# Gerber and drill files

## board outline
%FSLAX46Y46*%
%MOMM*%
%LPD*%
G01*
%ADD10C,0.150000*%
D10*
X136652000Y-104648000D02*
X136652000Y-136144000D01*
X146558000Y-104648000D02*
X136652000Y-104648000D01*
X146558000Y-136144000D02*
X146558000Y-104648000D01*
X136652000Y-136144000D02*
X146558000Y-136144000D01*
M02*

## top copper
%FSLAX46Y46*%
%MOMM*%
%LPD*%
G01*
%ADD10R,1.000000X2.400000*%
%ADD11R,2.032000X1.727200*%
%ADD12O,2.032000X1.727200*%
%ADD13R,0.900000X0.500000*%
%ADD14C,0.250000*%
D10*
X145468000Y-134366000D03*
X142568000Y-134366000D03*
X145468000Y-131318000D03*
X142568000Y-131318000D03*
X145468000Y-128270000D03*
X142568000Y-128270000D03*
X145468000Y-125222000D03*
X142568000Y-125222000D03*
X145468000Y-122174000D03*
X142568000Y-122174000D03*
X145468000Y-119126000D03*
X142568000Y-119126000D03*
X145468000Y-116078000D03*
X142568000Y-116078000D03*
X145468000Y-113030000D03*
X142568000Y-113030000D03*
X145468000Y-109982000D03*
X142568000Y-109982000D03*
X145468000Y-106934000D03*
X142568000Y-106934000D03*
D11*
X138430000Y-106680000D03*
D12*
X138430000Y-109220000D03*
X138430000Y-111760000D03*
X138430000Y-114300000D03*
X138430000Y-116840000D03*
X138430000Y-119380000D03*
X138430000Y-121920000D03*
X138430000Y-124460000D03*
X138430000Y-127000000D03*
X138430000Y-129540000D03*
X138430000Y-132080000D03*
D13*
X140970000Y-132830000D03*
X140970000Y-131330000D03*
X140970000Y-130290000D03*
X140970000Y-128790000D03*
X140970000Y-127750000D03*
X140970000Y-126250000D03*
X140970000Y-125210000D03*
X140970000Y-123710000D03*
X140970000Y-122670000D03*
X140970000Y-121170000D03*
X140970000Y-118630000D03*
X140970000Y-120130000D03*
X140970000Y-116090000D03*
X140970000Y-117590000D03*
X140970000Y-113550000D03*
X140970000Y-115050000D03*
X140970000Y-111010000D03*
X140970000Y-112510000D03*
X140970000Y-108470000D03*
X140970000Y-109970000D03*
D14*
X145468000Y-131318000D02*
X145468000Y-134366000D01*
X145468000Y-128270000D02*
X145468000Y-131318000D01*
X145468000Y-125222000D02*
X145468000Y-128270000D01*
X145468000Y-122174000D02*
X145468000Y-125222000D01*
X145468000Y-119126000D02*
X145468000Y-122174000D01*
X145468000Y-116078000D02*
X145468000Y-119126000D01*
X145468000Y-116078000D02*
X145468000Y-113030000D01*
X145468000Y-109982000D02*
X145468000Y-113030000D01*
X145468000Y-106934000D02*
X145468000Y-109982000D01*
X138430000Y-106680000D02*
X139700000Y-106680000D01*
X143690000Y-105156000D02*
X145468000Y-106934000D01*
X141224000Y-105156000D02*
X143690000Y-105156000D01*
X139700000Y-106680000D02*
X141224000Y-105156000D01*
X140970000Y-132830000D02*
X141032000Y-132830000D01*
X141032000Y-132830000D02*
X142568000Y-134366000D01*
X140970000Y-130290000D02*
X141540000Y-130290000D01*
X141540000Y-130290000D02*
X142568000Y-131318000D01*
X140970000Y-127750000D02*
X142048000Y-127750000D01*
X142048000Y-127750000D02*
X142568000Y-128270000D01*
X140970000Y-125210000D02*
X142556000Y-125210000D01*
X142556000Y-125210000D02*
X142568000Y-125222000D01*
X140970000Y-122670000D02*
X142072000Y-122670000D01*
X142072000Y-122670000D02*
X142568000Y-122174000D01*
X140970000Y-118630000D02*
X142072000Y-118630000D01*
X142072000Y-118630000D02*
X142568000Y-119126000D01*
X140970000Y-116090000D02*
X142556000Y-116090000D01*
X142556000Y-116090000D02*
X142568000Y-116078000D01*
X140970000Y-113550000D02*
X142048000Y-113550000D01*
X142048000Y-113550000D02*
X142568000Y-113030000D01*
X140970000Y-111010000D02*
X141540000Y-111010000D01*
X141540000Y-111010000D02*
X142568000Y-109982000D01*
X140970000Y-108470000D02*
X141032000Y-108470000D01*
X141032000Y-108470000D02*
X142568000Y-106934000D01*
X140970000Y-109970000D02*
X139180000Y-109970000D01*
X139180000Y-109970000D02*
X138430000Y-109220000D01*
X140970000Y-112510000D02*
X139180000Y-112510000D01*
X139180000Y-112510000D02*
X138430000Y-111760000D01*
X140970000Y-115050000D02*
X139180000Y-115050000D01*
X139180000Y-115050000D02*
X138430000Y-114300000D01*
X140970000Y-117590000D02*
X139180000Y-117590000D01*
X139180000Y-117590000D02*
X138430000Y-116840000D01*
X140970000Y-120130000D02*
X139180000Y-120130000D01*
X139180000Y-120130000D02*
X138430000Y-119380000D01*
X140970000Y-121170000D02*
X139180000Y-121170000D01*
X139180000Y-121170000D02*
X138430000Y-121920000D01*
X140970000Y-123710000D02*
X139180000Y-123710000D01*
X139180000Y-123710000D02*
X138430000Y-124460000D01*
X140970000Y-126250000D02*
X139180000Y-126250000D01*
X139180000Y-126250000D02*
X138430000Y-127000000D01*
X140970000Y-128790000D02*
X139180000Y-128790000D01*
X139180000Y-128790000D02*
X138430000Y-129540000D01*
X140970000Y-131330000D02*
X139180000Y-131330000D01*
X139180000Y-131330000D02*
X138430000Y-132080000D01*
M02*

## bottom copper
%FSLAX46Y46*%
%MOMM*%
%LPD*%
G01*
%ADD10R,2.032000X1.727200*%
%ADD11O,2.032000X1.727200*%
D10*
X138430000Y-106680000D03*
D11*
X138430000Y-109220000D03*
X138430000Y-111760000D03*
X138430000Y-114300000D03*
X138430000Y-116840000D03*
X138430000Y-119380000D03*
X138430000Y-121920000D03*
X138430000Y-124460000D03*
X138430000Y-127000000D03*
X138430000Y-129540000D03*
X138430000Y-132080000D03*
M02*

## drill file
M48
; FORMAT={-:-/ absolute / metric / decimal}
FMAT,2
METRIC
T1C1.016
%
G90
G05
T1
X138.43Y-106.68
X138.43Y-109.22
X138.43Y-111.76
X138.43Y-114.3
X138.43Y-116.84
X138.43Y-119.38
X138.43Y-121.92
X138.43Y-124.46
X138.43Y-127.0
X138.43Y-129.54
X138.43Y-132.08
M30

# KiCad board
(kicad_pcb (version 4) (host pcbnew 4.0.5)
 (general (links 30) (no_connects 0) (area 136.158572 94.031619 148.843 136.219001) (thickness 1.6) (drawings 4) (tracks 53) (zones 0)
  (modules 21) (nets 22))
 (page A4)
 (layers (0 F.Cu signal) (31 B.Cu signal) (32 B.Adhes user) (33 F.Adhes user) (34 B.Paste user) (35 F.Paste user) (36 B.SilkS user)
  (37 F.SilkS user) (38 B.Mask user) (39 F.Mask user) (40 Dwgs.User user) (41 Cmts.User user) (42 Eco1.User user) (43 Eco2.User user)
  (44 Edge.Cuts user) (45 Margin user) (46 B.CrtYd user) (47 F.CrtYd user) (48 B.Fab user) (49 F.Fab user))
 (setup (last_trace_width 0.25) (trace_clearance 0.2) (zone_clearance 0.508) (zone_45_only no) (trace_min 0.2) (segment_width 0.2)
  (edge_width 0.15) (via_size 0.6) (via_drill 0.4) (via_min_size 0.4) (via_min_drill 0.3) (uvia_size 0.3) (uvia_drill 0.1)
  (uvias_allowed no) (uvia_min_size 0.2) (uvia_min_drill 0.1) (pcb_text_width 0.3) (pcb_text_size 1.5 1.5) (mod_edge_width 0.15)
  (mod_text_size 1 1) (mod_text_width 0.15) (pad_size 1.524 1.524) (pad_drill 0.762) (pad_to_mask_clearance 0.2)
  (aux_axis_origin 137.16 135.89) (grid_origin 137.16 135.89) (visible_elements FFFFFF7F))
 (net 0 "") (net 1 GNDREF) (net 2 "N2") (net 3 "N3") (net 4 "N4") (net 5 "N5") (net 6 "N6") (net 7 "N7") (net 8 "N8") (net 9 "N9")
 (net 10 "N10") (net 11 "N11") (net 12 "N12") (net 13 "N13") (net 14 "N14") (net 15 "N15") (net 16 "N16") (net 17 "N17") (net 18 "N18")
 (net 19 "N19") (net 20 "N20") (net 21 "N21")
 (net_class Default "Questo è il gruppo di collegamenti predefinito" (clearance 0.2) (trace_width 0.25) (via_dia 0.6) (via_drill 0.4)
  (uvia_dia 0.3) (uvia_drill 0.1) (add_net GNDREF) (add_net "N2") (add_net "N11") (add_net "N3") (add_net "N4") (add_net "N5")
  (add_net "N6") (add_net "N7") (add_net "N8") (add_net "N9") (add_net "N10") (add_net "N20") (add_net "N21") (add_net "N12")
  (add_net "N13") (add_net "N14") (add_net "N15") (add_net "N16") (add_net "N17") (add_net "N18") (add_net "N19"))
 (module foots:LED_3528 (layer F.Cu) (at 144.018 134.366 90)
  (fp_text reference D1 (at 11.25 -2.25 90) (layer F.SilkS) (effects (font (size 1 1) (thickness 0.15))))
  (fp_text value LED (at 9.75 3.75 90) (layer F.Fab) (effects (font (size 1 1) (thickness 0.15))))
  (pad 1 smd rect (at 0 1.45 90) (size 2.4 1) (layers F.Cu F.Paste F.Mask) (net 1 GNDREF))
  (pad 2 smd rect (at 0 -1.45 90) (size 2.4 1) (layers F.Cu F.Paste F.Mask) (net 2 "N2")))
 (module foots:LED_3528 (layer F.Cu) (at 144.018 131.318 90)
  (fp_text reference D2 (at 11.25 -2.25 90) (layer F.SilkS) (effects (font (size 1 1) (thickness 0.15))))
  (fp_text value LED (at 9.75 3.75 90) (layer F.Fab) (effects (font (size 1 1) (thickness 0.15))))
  (pad 1 smd rect (at 0 1.45 90) (size 2.4 1) (layers F.Cu F.Paste F.Mask) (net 1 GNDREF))
  (pad 2 smd rect (at 0 -1.45 90) (size 2.4 1) (layers F.Cu F.Paste F.Mask) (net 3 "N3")))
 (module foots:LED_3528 (layer F.Cu) (at 144.018 128.27 90)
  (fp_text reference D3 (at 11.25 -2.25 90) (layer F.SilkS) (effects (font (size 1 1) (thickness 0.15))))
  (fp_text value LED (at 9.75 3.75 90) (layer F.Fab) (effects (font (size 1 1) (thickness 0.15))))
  (pad 1 smd rect (at 0 1.45 90) (size 2.4 1) (layers F.Cu F.Paste F.Mask) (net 1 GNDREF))
  (pad 2 smd rect (at 0 -1.45 90) (size 2.4 1) (layers F.Cu F.Paste F.Mask) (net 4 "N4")))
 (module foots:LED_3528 (layer F.Cu) (at 144.018 125.222 90)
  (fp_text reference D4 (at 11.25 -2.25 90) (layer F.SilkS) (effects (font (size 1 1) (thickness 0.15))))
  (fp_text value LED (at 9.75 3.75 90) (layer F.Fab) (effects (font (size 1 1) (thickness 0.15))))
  (pad 1 smd rect (at 0 1.45 90) (size 2.4 1) (layers F.Cu F.Paste F.Mask) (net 1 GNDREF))
  (pad 2 smd rect (at 0 -1.45 90) (size 2.4 1) (layers F.Cu F.Paste F.Mask) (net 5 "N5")))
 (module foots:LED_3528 (layer F.Cu) (at 144.018 122.174 90)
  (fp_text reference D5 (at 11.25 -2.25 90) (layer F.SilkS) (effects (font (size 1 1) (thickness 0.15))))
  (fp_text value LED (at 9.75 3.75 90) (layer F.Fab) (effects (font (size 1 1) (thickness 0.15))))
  (pad 1 smd rect (at 0 1.45 90) (size 2.4 1) (layers F.Cu F.Paste F.Mask) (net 1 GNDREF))
  (pad 2 smd rect (at 0 -1.45 90) (size 2.4 1) (layers F.Cu F.Paste F.Mask) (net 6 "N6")))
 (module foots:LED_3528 (layer F.Cu) (at 144.018 119.126 90)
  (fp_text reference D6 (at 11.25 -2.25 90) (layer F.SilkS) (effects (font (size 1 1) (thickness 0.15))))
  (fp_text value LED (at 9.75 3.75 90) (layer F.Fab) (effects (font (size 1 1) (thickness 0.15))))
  (pad 1 smd rect (at 0 1.45 90) (size 2.4 1) (layers F.Cu F.Paste F.Mask) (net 1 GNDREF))
  (pad 2 smd rect (at 0 -1.45 90) (size 2.4 1) (layers F.Cu F.Paste F.Mask) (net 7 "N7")))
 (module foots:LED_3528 (layer F.Cu) (at 144.018 116.078 90)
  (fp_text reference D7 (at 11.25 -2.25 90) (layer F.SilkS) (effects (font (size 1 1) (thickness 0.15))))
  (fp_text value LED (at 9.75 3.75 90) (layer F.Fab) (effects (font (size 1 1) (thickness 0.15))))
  (pad 1 smd rect (at 0 1.45 90) (size 2.4 1) (layers F.Cu F.Paste F.Mask) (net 1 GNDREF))
  (pad 2 smd rect (at 0 -1.45 90) (size 2.4 1) (layers F.Cu F.Paste F.Mask) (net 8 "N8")))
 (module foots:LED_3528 (layer F.Cu) (at 144.018 113.03 90)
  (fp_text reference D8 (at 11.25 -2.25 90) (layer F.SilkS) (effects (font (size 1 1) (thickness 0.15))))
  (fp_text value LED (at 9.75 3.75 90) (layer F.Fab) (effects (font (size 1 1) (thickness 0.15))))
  (pad 1 smd rect (at 0 1.45 90) (size 2.4 1) (layers F.Cu F.Paste F.Mask) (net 1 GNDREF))
  (pad 2 smd rect (at 0 -1.45 90) (size 2.4 1) (layers F.Cu F.Paste F.Mask) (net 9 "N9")))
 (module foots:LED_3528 (layer F.Cu) (at 144.018 109.982 90)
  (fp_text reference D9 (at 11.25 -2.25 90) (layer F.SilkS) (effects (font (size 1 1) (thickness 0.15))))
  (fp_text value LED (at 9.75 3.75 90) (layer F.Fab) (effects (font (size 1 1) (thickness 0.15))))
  (pad 1 smd rect (at 0 1.45 90) (size 2.4 1) (layers F.Cu F.Paste F.Mask) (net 1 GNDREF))
  (pad 2 smd rect (at 0 -1.45 90) (size 2.4 1) (layers F.Cu F.Paste F.Mask) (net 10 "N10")))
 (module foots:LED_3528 (layer F.Cu) (at 144.018 106.934 90)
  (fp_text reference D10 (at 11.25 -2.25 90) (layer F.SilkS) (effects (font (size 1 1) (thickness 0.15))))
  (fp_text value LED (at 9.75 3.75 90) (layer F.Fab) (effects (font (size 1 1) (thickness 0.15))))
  (pad 1 smd rect (at 0 1.45 90) (size 2.4 1) (layers F.Cu F.Paste F.Mask) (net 1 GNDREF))
  (pad 2 smd rect (at 0 -1.45 90) (size 2.4 1) (layers F.Cu F.Paste F.Mask) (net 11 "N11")))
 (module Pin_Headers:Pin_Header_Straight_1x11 (layer F.Cu) (at 138.43 106.68)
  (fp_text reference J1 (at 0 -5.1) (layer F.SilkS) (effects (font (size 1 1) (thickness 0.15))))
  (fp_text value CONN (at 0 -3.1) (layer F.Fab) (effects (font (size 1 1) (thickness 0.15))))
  (pad 1 thru_hole rect (at 0 0) (size 2.032 1.7272) (drill 1.016) (layers *.Cu *.Mask) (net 1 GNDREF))
  (pad 2 thru_hole oval (at 0 2.54) (size 2.032 1.7272) (drill 1.016) (layers *.Cu *.Mask) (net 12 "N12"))
  (pad 3 thru_hole oval (at 0 5.08) (size 2.032 1.7272) (drill 1.016) (layers *.Cu *.Mask) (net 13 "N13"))
  (pad 4 thru_hole oval (at 0 7.62) (size 2.032 1.7272) (drill 1.016) (layers *.Cu *.Mask) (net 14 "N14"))
  (pad 5 thru_hole oval (at 0 10.16) (size 2.032 1.7272) (drill 1.016) (layers *.Cu *.Mask) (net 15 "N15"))
  (pad 6 thru_hole oval (at 0 12.7) (size 2.032 1.7272) (drill 1.016) (layers *.Cu *.Mask) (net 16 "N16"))
  (pad 7 thru_hole oval (at 0 15.24) (size 2.032 1.7272) (drill 1.016) (layers *.Cu *.Mask) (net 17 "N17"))
  (pad 8 thru_hole oval (at 0 17.78) (size 2.032 1.7272) (drill 1.016) (layers *.Cu *.Mask) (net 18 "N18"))
  (pad 9 thru_hole oval (at 0 20.32) (size 2.032 1.7272) (drill 1.016) (layers *.Cu *.Mask) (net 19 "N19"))
  (pad 10 thru_hole oval (at 0 22.86) (size 2.032 1.7272) (drill 1.016) (layers *.Cu *.Mask) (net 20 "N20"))
  (pad 11 thru_hole oval (at 0 25.4) (size 2.032 1.7272) (drill 1.016) (layers *.Cu *.Mask) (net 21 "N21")))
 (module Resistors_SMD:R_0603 (layer F.Cu) (at 140.97 132.08 90)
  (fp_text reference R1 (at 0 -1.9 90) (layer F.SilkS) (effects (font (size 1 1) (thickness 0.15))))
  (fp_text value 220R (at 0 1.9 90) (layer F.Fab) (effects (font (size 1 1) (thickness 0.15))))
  (pad 1 smd rect (at -0.75 0 90) (size 0.5 0.9) (layers F.Cu F.Paste F.Mask) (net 2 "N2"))
  (pad 2 smd rect (at 0.75 0 90) (size 0.5 0.9) (layers F.Cu F.Paste F.Mask) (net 21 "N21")))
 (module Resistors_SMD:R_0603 (layer F.Cu) (at 140.97 129.54 90)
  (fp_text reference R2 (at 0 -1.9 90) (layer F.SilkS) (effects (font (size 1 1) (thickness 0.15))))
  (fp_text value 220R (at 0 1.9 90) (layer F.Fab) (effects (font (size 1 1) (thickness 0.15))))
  (pad 1 smd rect (at -0.75 0 90) (size 0.5 0.9) (layers F.Cu F.Paste F.Mask) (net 3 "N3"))
  (pad 2 smd rect (at 0.75 0 90) (size 0.5 0.9) (layers F.Cu F.Paste F.Mask) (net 20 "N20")))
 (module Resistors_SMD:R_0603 (layer F.Cu) (at 140.97 127 90)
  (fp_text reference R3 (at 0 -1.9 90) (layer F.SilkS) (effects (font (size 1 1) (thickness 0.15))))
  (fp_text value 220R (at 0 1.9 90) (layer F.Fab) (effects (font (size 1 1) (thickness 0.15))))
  (pad 1 smd rect (at -0.75 0 90) (size 0.5 0.9) (layers F.Cu F.Paste F.Mask) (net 4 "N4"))
  (pad 2 smd rect (at 0.75 0 90) (size 0.5 0.9) (layers F.Cu F.Paste F.Mask) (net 19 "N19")))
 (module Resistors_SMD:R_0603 (layer F.Cu) (at 140.97 124.46 90)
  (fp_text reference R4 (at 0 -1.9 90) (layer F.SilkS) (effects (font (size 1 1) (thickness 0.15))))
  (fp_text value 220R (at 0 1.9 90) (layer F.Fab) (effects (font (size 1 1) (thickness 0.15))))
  (pad 1 smd rect (at -0.75 0 90) (size 0.5 0.9) (layers F.Cu F.Paste F.Mask) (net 5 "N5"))
  (pad 2 smd rect (at 0.75 0 90) (size 0.5 0.9) (layers F.Cu F.Paste F.Mask) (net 18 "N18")))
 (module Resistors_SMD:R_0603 (layer F.Cu) (at 140.97 121.92 90)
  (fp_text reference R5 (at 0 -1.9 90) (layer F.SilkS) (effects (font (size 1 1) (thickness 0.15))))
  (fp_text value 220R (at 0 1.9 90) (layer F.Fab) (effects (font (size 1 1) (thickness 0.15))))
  (pad 1 smd rect (at -0.75 0 90) (size 0.5 0.9) (layers F.Cu F.Paste F.Mask) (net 6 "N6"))
  (pad 2 smd rect (at 0.75 0 90) (size 0.5 0.9) (layers F.Cu F.Paste F.Mask) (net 17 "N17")))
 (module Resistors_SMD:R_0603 (layer F.Cu) (at 140.97 119.38 270)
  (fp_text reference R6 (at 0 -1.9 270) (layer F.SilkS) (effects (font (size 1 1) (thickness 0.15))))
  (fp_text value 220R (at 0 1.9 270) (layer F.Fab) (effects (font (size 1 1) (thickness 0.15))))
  (pad 1 smd rect (at -0.75 0 270) (size 0.5 0.9) (layers F.Cu F.Paste F.Mask) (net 7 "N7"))
  (pad 2 smd rect (at 0.75 0 270) (size 0.5 0.9) (layers F.Cu F.Paste F.Mask) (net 16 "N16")))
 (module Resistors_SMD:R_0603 (layer F.Cu) (at 140.97 116.84 270)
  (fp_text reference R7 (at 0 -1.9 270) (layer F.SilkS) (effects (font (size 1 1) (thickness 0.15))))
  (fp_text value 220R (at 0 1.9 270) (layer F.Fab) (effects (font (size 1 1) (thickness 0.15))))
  (pad 1 smd rect (at -0.75 0 270) (size 0.5 0.9) (layers F.Cu F.Paste F.Mask) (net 8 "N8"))
  (pad 2 smd rect (at 0.75 0 270) (size 0.5 0.9) (layers F.Cu F.Paste F.Mask) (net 15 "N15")))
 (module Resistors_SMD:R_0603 (layer F.Cu) (at 140.97 114.3 270)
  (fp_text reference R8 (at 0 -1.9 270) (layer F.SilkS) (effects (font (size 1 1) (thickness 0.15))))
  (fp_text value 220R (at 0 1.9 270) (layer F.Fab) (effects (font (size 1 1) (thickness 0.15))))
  (pad 1 smd rect (at -0.75 0 270) (size 0.5 0.9) (layers F.Cu F.Paste F.Mask) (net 9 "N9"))
  (pad 2 smd rect (at 0.75 0 270) (size 0.5 0.9) (layers F.Cu F.Paste F.Mask) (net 14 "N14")))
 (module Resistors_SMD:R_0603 (layer F.Cu) (at 140.97 111.76 270)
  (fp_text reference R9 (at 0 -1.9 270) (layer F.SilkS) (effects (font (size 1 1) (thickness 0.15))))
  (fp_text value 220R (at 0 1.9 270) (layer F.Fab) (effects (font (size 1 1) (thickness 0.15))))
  (pad 1 smd rect (at -0.75 0 270) (size 0.5 0.9) (layers F.Cu F.Paste F.Mask) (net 10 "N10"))
  (pad 2 smd rect (at 0.75 0 270) (size 0.5 0.9) (layers F.Cu F.Paste F.Mask) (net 13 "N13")))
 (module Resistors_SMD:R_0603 (layer F.Cu) (at 140.97 109.22 270)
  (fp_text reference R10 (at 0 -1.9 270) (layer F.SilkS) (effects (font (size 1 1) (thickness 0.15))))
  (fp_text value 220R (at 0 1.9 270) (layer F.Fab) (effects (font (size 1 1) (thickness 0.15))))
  (pad 1 smd rect (at -0.75 0 270) (size 0.5 0.9) (layers F.Cu F.Paste F.Mask) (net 11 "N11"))
  (pad 2 smd rect (at 0.75 0 270) (size 0.5 0.9) (layers F.Cu F.Paste F.Mask) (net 12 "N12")))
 (gr_line (start 136.652 104.648) (end 136.652 136.144) (angle 90) (layer Edge.Cuts) (width 0.15))
 (gr_line (start 146.558 104.648) (end 136.652 104.648) (angle 90) (layer Edge.Cuts) (width 0.15))
 (gr_line (start 146.558 136.144) (end 146.558 104.648) (angle 90) (layer Edge.Cuts) (width 0.15))
 (gr_line (start 136.652 136.144) (end 146.558 136.144) (angle 90) (layer Edge.Cuts) (width 0.15))
 (segment (start 145.468 131.318) (end 145.468 134.366) (width 0.25) (layer F.Cu) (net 1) (status C00000))
 (segment (start 145.468 128.27) (end 145.468 131.318) (width 0.25) (layer F.Cu) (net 1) (status C00000))
 (segment (start 145.468 125.222) (end 145.468 128.27) (width 0.25) (layer F.Cu) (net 1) (status C00000))
 (segment (start 145.468 122.174) (end 145.468 125.222) (width 0.25) (layer F.Cu) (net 1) (status C00000))
 (segment (start 145.468 119.126) (end 145.468 122.174) (width 0.25) (layer F.Cu) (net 1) (status C00000))
 (segment (start 145.468 116.078) (end 145.468 119.126) (width 0.25) (layer F.Cu) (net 1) (status C00000))
 (segment (start 145.468 116.078) (end 145.468 113.03) (width 0.25) (layer F.Cu) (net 1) (status C00000))
 (segment (start 145.468 109.982) (end 145.468 113.03) (width 0.25) (layer F.Cu) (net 1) (status C00000))
 (segment (start 145.468 106.934) (end 145.468 109.982) (width 0.25) (layer F.Cu) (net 1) (status C00000))
 (segment (start 138.43 106.68) (end 139.7 106.68) (width 0.25) (layer F.Cu) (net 1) (status 400000))
 (segment (start 143.69 105.156) (end 145.468 106.934) (width 0.25) (layer F.Cu) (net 1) (status 800000))
 (segment (start 141.224 105.156) (end 143.69 105.156) (width 0.25) (layer F.Cu) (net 1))
 (segment (start 139.7 106.68) (end 141.224 105.156) (width 0.25) (layer F.Cu) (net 1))
 (segment (start 140.97 132.83) (end 141.032 132.83) (width 0.25) (layer F.Cu) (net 2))
 (segment (start 141.032 132.83) (end 142.568 134.366) (width 0.25) (layer F.Cu) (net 2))
 (segment (start 140.97 130.29) (end 141.54 130.29) (width 0.25) (layer F.Cu) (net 3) (status 400000))
 (segment (start 141.54 130.29) (end 142.568 131.318) (width 0.25) (layer F.Cu) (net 3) (status 800000))
 (segment (start 140.97 127.75) (end 142.048 127.75) (width 0.25) (layer F.Cu) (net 4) (status 400000))
 (segment (start 142.048 127.75) (end 142.568 128.27) (width 0.25) (layer F.Cu) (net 4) (status 800000))
 (segment (start 140.97 125.21) (end 142.556 125.21) (width 0.25) (layer F.Cu) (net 5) (status C00000))
 (segment (start 142.556 125.21) (end 142.568 125.222) (width 0.25) (layer F.Cu) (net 5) (status C00000))
 (segment (start 140.97 122.67) (end 142.072 122.67) (width 0.25) (layer F.Cu) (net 6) (status C00000))
 (segment (start 142.072 122.67) (end 142.568 122.174) (width 0.25) (layer F.Cu) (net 6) (status C00000))
 (segment (start 140.97 118.63) (end 142.072 118.63) (width 0.25) (layer F.Cu) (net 7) (status C00000))
 (segment (start 142.072 118.63) (end 142.568 119.126) (width 0.25) (layer F.Cu) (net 7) (status C00000))
 (segment (start 140.97 116.09) (end 142.556 116.09) (width 0.25) (layer F.Cu) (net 8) (status C00000))
 (segment (start 142.556 116.09) (end 142.568 116.078) (width 0.25) (layer F.Cu) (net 8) (status C00000))
 (segment (start 140.97 113.55) (end 142.048 113.55) (width 0.25) (layer F.Cu) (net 9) (status 400000))
 (segment (start 142.048 113.55) (end 142.568 113.03) (width 0.25) (layer F.Cu) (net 9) (status 800000))
 (segment (start 140.97 111.01) (end 141.54 111.01) (width 0.25) (layer F.Cu) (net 10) (status 400000))
 (segment (start 141.54 111.01) (end 142.568 109.982) (width 0.25) (layer F.Cu) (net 10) (status 800000))
 (segment (start 140.97 108.47) (end 141.032 108.47) (width 0.25) (layer F.Cu) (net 11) (status C00000))
 (segment (start 141.032 108.47) (end 142.568 106.934) (width 0.25) (layer F.Cu) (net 11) (status C00000))
 (segment (start 140.97 109.97) (end 139.18 109.97) (width 0.25) (layer F.Cu) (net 12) (status 400000))
 (segment (start 139.18 109.97) (end 138.43 109.22) (width 0.25) (layer F.Cu) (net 12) (status 800000))
 (segment (start 140.97 112.51) (end 139.18 112.51) (width 0.25) (layer F.Cu) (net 13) (status 400000))
 (segment (start 139.18 112.51) (end 138.43 111.76) (width 0.25) (layer F.Cu) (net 13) (status 800000))
 (segment (start 140.97 115.05) (end 139.18 115.05) (width 0.25) (layer F.Cu) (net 14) (status 400000))
 (segment (start 139.18 115.05) (end 138.43 114.3) (width 0.25) (layer F.Cu) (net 14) (status 800000))
 (segment (start 140.97 117.59) (end 139.18 117.59) (width 0.25) (layer F.Cu) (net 15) (status 400000))
 (segment (start 139.18 117.59) (end 138.43 116.84) (width 0.25) (layer F.Cu) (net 15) (status 800000))
 (segment (start 140.97 120.13) (end 139.18 120.13) (width 0.25) (layer F.Cu) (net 16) (status 400000))
 (segment (start 139.18 120.13) (end 138.43 119.38) (width 0.25) (layer F.Cu) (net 16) (status 800000))
 (segment (start 140.97 121.17) (end 139.18 121.17) (width 0.25) (layer F.Cu) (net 17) (status 400000))
 (segment (start 139.18 121.17) (end 138.43 121.92) (width 0.25) (layer F.Cu) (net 17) (status 800000))
 (segment (start 140.97 123.71) (end 139.18 123.71) (width 0.25) (layer F.Cu) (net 18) (status 400000))
 (segment (start 139.18 123.71) (end 138.43 124.46) (width 0.25) (layer F.Cu) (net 18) (status 800000))
 (segment (start 140.97 126.25) (end 139.18 126.25) (width 0.25) (layer F.Cu) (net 19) (status 400000))
 (segment (start 139.18 126.25) (end 138.43 127) (width 0.25) (layer F.Cu) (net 19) (status 800000))
 (segment (start 140.97 128.79) (end 139.18 128.79) (width 0.25) (layer F.Cu) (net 20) (status 400000))
 (segment (start 139.18 128.79) (end 138.43 129.54) (width 0.25) (layer F.Cu) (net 20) (status 800000))
 (segment (start 140.97 131.33) (end 139.18 131.33) (width 0.25) (layer F.Cu) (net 21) (status 400000))
 (segment (start 139.18 131.33) (end 138.43 132.08) (width 0.25) (layer F.Cu) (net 21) (status 800000)))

